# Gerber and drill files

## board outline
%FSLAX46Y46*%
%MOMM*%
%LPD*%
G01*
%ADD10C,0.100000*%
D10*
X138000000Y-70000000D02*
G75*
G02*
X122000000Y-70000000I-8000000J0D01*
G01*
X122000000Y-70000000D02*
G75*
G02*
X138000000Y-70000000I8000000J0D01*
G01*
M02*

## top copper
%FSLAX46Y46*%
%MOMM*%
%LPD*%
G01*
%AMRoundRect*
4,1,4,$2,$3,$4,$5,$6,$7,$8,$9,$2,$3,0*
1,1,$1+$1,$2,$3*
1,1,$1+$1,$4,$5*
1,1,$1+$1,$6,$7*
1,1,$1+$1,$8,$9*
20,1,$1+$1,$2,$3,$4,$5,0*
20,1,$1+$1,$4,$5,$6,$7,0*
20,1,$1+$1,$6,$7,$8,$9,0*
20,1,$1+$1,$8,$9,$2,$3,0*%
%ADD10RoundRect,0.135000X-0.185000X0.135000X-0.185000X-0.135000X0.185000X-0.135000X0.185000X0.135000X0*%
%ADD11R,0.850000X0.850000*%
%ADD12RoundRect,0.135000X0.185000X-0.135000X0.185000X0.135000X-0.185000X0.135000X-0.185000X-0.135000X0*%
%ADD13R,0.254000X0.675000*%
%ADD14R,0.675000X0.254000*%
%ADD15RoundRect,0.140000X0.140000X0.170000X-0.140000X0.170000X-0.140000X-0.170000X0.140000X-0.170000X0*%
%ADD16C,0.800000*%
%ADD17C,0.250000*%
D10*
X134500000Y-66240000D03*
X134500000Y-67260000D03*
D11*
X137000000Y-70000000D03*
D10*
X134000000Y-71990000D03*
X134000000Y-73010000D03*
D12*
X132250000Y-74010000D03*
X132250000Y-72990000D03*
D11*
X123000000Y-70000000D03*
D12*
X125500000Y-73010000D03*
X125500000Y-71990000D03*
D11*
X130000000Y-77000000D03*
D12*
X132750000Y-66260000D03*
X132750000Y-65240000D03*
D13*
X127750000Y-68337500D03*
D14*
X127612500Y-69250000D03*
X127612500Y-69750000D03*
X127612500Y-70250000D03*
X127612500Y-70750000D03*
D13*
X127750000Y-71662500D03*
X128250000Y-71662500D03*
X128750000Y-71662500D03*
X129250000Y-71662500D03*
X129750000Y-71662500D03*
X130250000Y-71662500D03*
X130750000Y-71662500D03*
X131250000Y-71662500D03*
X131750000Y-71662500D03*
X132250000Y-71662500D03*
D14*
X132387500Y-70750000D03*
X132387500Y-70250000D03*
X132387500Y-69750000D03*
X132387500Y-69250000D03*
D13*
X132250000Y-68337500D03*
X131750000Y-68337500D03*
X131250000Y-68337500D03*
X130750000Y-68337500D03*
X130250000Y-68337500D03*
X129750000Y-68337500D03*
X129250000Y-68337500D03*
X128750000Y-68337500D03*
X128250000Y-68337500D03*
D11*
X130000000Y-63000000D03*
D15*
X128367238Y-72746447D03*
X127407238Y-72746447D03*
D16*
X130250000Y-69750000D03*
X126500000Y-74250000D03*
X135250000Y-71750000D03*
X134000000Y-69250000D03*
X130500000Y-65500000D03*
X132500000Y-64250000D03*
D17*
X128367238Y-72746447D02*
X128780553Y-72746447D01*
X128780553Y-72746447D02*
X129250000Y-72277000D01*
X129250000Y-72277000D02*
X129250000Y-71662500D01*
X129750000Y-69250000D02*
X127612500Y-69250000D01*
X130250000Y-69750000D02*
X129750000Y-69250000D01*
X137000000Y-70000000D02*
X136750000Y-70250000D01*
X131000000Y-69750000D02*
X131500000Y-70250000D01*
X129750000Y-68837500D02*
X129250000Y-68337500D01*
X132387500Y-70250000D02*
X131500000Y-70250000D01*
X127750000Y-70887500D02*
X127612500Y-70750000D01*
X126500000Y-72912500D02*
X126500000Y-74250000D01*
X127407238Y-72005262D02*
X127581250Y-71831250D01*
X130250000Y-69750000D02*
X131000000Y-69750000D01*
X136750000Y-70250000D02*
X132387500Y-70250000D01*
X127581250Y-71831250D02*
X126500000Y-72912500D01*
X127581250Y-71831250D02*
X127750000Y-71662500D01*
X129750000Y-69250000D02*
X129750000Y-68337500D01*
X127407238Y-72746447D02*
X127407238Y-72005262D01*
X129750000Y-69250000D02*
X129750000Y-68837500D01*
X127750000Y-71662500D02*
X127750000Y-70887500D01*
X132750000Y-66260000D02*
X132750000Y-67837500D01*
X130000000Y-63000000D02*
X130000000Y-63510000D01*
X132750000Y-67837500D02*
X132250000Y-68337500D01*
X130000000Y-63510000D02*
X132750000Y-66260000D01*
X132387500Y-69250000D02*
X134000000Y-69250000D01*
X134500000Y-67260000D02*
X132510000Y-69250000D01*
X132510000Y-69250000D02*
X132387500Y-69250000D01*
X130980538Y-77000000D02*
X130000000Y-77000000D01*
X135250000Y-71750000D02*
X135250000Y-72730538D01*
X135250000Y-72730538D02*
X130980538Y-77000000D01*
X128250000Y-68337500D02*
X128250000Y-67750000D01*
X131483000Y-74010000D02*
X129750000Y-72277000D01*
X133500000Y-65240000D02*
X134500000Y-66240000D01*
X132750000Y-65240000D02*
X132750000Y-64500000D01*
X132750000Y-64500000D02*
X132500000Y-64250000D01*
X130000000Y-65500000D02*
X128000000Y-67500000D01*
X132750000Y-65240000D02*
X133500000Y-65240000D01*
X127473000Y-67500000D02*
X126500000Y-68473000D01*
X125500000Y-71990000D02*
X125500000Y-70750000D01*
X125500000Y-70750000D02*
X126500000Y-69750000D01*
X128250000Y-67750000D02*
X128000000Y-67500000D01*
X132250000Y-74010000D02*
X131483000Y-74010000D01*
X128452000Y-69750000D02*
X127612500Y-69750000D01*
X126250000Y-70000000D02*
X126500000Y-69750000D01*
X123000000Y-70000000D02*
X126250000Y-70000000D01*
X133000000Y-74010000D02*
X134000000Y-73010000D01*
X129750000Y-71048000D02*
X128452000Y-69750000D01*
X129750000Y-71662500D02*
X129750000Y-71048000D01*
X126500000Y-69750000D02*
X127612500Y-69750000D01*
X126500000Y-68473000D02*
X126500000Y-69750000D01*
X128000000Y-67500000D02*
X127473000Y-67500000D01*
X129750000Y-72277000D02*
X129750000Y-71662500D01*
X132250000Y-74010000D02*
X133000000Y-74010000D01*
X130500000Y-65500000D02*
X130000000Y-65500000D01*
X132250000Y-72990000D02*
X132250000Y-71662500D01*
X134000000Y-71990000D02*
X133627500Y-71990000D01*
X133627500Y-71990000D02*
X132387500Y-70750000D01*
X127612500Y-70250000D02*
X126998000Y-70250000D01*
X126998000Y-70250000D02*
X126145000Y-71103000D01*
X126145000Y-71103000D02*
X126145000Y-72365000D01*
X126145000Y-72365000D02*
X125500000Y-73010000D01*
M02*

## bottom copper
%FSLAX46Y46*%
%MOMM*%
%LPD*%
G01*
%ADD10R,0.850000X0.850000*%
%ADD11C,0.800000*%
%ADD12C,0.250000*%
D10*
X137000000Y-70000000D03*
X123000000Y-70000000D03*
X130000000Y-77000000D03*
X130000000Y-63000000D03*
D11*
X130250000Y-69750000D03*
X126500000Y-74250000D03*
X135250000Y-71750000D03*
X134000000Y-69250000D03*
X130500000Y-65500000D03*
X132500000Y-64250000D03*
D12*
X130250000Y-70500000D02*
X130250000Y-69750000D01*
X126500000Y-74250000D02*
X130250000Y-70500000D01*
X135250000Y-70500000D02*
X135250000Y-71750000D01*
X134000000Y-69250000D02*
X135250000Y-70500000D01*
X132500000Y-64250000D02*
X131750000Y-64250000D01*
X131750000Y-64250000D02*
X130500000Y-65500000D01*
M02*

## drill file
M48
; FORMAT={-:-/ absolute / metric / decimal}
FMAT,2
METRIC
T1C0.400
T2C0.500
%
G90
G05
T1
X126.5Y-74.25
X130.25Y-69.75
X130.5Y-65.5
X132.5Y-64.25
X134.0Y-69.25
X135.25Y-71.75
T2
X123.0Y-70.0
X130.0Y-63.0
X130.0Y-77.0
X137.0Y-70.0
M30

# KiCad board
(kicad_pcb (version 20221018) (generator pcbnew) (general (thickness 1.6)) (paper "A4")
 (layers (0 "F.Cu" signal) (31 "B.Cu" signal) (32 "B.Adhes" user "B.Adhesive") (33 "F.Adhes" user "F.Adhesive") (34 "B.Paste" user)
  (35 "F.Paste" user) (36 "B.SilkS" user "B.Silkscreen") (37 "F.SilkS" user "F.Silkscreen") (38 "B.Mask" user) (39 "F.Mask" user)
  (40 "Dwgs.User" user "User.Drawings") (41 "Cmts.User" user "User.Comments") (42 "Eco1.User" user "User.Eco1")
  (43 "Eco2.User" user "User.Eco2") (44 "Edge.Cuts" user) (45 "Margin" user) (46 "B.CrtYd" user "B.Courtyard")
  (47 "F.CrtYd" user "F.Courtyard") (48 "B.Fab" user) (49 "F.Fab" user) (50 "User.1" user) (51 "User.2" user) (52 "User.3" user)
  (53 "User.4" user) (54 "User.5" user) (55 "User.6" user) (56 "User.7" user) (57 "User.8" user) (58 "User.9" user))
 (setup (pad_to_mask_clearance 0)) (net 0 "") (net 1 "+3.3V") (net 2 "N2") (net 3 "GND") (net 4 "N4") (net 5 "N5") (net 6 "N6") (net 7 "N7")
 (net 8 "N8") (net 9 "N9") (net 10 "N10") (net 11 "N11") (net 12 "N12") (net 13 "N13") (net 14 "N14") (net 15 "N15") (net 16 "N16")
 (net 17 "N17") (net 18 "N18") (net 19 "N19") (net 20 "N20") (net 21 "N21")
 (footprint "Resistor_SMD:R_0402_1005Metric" (layer "F.Cu") (at 134.5 66.75 -90)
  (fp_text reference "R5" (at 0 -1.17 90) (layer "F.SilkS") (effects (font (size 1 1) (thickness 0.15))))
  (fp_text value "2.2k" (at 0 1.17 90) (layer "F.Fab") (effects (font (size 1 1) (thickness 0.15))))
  (pad "1" smd roundrect (at -0.51 0 270) (size 0.54 0.64) (layers "F.Cu" "F.Paste" "F.Mask") (roundrect_rratio 0.25) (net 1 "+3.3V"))
  (pad "2" smd roundrect (at 0.51 0 270) (size 0.54 0.64) (layers "F.Cu" "F.Paste" "F.Mask") (roundrect_rratio 0.25) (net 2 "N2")))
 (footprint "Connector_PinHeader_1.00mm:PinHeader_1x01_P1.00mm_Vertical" (layer "F.Cu") (at 137 70 -90)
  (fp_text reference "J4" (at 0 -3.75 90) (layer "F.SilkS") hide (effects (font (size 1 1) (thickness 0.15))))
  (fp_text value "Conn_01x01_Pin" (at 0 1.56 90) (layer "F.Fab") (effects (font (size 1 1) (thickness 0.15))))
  (pad "1" thru_hole rect (at 0 0 270) (size 0.85 0.85) (drill 0.5) (layers "*.Cu" "*.Mask") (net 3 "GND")))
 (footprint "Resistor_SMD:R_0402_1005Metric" (layer "F.Cu") (at 134 72.5 -90)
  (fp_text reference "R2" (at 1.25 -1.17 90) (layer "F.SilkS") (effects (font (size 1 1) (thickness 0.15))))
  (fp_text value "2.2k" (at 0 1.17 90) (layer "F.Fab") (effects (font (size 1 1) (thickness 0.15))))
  (pad "1" smd roundrect (at -0.51 0 270) (size 0.54 0.64) (layers "F.Cu" "F.Paste" "F.Mask") (roundrect_rratio 0.25) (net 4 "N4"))
  (pad "2" smd roundrect (at 0.51 0 270) (size 0.54 0.64) (layers "F.Cu" "F.Paste" "F.Mask") (roundrect_rratio 0.25) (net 1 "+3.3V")))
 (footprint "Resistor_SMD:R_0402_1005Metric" (layer "F.Cu") (at 132.25 73.5 90)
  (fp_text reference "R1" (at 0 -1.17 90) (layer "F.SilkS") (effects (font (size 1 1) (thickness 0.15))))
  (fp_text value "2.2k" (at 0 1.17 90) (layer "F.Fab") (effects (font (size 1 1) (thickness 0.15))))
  (pad "1" smd roundrect (at -0.51 0 90) (size 0.54 0.64) (layers "F.Cu" "F.Paste" "F.Mask") (roundrect_rratio 0.25) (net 1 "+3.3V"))
  (pad "2" smd roundrect (at 0.51 0 90) (size 0.54 0.64) (layers "F.Cu" "F.Paste" "F.Mask") (roundrect_rratio 0.25) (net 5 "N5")))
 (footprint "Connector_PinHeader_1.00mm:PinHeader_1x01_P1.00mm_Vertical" (layer "F.Cu") (at 123 70 90)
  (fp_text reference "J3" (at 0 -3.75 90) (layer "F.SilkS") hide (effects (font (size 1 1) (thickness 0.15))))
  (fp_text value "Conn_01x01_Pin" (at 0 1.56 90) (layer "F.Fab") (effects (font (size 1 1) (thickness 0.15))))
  (pad "1" thru_hole rect (at 0 0 90) (size 0.85 0.85) (drill 0.5) (layers "*.Cu" "*.Mask") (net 1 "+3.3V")))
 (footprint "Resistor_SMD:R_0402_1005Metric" (layer "F.Cu") (at 125.5 72.5 90)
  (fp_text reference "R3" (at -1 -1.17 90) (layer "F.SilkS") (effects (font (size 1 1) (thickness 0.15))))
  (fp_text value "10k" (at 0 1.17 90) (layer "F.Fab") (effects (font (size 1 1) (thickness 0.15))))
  (pad "1" smd roundrect (at -0.51 0 90) (size 0.54 0.64) (layers "F.Cu" "F.Paste" "F.Mask") (roundrect_rratio 0.25) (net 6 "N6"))
  (pad "2" smd roundrect (at 0.51 0 90) (size 0.54 0.64) (layers "F.Cu" "F.Paste" "F.Mask") (roundrect_rratio 0.25) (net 1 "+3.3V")))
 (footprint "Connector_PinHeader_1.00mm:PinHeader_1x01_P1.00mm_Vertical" (layer "F.Cu") (at 130 77 180)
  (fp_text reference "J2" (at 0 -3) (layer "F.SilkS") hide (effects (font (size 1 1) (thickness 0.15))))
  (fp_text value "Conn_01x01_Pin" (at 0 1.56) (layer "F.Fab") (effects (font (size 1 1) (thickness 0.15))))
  (pad "1" thru_hole rect (at 0 0 180) (size 0.85 0.85) (drill 0.5) (layers "*.Cu" "*.Mask") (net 2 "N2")))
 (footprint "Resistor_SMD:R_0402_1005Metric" (layer "F.Cu") (at 132.75 65.75 90)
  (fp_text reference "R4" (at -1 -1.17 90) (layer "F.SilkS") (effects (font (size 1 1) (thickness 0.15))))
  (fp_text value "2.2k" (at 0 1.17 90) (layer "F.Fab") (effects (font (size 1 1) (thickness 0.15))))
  (pad "1" smd roundrect (at -0.51 0 90) (size 0.54 0.64) (layers "F.Cu" "F.Paste" "F.Mask") (roundrect_rratio 0.25) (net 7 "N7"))
  (pad "2" smd roundrect (at 0.51 0 90) (size 0.54 0.64) (layers "F.Cu" "F.Paste" "F.Mask") (roundrect_rratio 0.25) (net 1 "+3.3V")))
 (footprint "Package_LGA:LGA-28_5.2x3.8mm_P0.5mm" (layer "F.Cu") (at 130 70)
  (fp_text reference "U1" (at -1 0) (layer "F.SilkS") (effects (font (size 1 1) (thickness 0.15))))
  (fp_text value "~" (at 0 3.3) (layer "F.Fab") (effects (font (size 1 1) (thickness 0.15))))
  (pad "1" smd rect (at -2.25 -1.6625) (size 0.254 0.675) (layers "F.Cu" "F.Paste" "F.Mask") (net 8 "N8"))
  (pad "2" smd rect (at -2.3875 -0.75 90) (size 0.254 0.675) (layers "F.Cu" "F.Paste" "F.Mask") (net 3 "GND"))
  (pad "3" smd rect (at -2.3875 -0.25 90) (size 0.254 0.675) (layers "F.Cu" "F.Paste" "F.Mask") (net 1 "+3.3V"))
  (pad "4" smd rect (at -2.3875 0.25 90) (size 0.254 0.675) (layers "F.Cu" "F.Paste" "F.Mask") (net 6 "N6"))
  (pad "5" smd rect (at -2.3875 0.75 90) (size 0.254 0.675) (layers "F.Cu" "F.Paste" "F.Mask") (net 3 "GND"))
  (pad "6" smd rect (at -2.25 1.6625) (size 0.254 0.675) (layers "F.Cu" "F.Paste" "F.Mask") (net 3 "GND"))
  (pad "7" smd rect (at -1.75 1.6625) (size 0.254 0.675) (layers "F.Cu" "F.Paste" "F.Mask") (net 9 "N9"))
  (pad "8" smd rect (at -1.25 1.6625) (size 0.254 0.675) (layers "F.Cu" "F.Paste" "F.Mask") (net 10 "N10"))
  (pad "9" smd rect (at -0.75 1.6625) (size 0.254 0.675) (layers "F.Cu" "F.Paste" "F.Mask") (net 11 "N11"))
  (pad "10" smd rect (at -0.25 1.6625) (size 0.254 0.675) (layers "F.Cu" "F.Paste" "F.Mask") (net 1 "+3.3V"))
  (pad "11" smd rect (at 0.25 1.6625) (size 0.254 0.675) (layers "F.Cu" "F.Paste" "F.Mask") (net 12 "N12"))
  (pad "12" smd rect (at 0.75 1.6625) (size 0.254 0.675) (layers "F.Cu" "F.Paste" "F.Mask") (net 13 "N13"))
  (pad "13" smd rect (at 1.25 1.6625) (size 0.254 0.675) (layers "F.Cu" "F.Paste" "F.Mask") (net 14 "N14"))
  (pad "14" smd rect (at 1.75 1.6625) (size 0.254 0.675) (layers "F.Cu" "F.Paste" "F.Mask") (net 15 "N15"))
  (pad "15" smd rect (at 2.25 1.6625) (size 0.254 0.675) (layers "F.Cu" "F.Paste" "F.Mask") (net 5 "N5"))
  (pad "16" smd rect (at 2.3875 0.75 90) (size 0.254 0.675) (layers "F.Cu" "F.Paste" "F.Mask") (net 4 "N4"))
  (pad "17" smd rect (at 2.3875 0.25 90) (size 0.254 0.675) (layers "F.Cu" "F.Paste" "F.Mask") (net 3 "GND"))
  (pad "18" smd rect (at 2.3875 -0.25 90) (size 0.254 0.675) (layers "F.Cu" "F.Paste" "F.Mask") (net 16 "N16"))
  (pad "19" smd rect (at 2.3875 -0.75 90) (size 0.254 0.675) (layers "F.Cu" "F.Paste" "F.Mask") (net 2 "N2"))
  (pad "20" smd rect (at 2.25 -1.6625) (size 0.254 0.675) (layers "F.Cu" "F.Paste" "F.Mask") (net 7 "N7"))
  (pad "21" smd rect (at 1.75 -1.6625) (size 0.254 0.675) (layers "F.Cu" "F.Paste" "F.Mask") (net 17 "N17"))
  (pad "22" smd rect (at 1.25 -1.6625) (size 0.254 0.675) (layers "F.Cu" "F.Paste" "F.Mask") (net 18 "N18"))
  (pad "23" smd rect (at 0.75 -1.6625) (size 0.254 0.675) (layers "F.Cu" "F.Paste" "F.Mask") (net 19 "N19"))
  (pad "24" smd rect (at 0.25 -1.6625) (size 0.254 0.675) (layers "F.Cu" "F.Paste" "F.Mask") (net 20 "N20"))
  (pad "25" smd rect (at -0.25 -1.6625) (size 0.254 0.675) (layers "F.Cu" "F.Paste" "F.Mask") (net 3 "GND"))
  (pad "26" smd rect (at -0.75 -1.6625) (size 0.254 0.675) (layers "F.Cu" "F.Paste" "F.Mask") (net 3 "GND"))
  (pad "27" smd rect (at -1.25 -1.6625) (size 0.254 0.675) (layers "F.Cu" "F.Paste" "F.Mask") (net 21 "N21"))
  (pad "28" smd rect (at -1.75 -1.6625) (size 0.254 0.675) (layers "F.Cu" "F.Paste" "F.Mask") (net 1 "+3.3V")))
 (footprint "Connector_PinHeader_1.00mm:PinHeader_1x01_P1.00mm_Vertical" (layer "F.Cu") (at 130 63)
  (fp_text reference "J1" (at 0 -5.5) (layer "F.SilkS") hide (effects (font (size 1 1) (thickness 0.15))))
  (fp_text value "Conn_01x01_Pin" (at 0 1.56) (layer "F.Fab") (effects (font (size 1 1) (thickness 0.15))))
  (pad "1" thru_hole rect (at 0 0) (size 0.85 0.85) (drill 0.5) (layers "*.Cu" "*.Mask") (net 7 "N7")))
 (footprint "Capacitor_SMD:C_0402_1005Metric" (layer "F.Cu") (at 127.887238 72.746447 180)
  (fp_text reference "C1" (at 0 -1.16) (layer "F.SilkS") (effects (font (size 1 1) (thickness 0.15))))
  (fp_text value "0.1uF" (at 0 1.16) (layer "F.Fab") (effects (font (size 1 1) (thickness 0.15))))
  (pad "1" smd roundrect (at -0.48 0 180) (size 0.56 0.62) (layers "F.Cu" "F.Paste" "F.Mask") (roundrect_rratio 0.25) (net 11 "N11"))
  (pad "2" smd roundrect (at 0.48 0 180) (size 0.56 0.62) (layers "F.Cu" "F.Paste" "F.Mask") (roundrect_rratio 0.25) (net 3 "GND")))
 (gr_circle (center 130 70) (end 138 70) (stroke (width 0.1) (type default)) (fill none) (layer "Edge.Cuts"))
 (segment (start 128.367238 72.746447) (end 128.780553 72.746447) (width 0.25) (layer "F.Cu") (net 11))
 (segment (start 128.780553 72.746447) (end 129.25 72.277) (width 0.25) (layer "F.Cu") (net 11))
 (segment (start 129.25 72.277) (end 129.25 71.6625) (width 0.25) (layer "F.Cu") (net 11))
 (segment (start 129.75 69.25) (end 127.6125 69.25) (width 0.25) (layer "F.Cu") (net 3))
 (segment (start 130.25 69.75) (end 129.75 69.25) (width 0.25) (layer "F.Cu") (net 3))
 (segment (start 137 70) (end 136.75 70.25) (width 0.25) (layer "F.Cu") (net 3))
 (segment (start 131 69.75) (end 131.5 70.25) (width 0.25) (layer "F.Cu") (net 3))
 (segment (start 129.75 68.8375) (end 129.25 68.3375) (width 0.25) (layer "F.Cu") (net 3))
 (segment (start 132.3875 70.25) (end 131.5 70.25) (width 0.25) (layer "F.Cu") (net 3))
 (segment (start 127.75 70.8875) (end 127.6125 70.75) (width 0.25) (layer "F.Cu") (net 3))
 (segment (start 126.5 72.9125) (end 126.5 74.25) (width 0.25) (layer "F.Cu") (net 3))
 (segment (start 127.407238 72.005262) (end 127.58125 71.83125) (width 0.25) (layer "F.Cu") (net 3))
 (segment (start 130.25 69.75) (end 131 69.75) (width 0.25) (layer "F.Cu") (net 3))
 (segment (start 136.75 70.25) (end 132.3875 70.25) (width 0.25) (layer "F.Cu") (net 3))
 (segment (start 127.58125 71.83125) (end 126.5 72.9125) (width 0.25) (layer "F.Cu") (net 3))
 (segment (start 127.58125 71.83125) (end 127.75 71.6625) (width 0.25) (layer "F.Cu") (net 3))
 (segment (start 129.75 69.25) (end 129.75 68.3375) (width 0.25) (layer "F.Cu") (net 3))
 (segment (start 127.407238 72.746447) (end 127.407238 72.005262) (width 0.25) (layer "F.Cu") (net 3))
 (segment (start 129.75 69.25) (end 129.75 68.8375) (width 0.25) (layer "F.Cu") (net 3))
 (segment (start 127.75 71.6625) (end 127.75 70.8875) (width 0.25) (layer "F.Cu") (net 3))
 (via (at 130.25 69.75) (size 0.8) (drill 0.4) (layers "F.Cu" "B.Cu") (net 3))
 (via (at 126.5 74.25) (size 0.8) (drill 0.4) (layers "F.Cu" "B.Cu") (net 3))
 (segment (start 130.25 70.5) (end 130.25 69.75) (width 0.25) (layer "B.Cu") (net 3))
 (segment (start 126.5 74.25) (end 130.25 70.5) (width 0.25) (layer "B.Cu") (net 3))
 (segment (start 132.75 66.26) (end 132.75 67.8375) (width 0.25) (layer "F.Cu") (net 7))
 (segment (start 130 63) (end 130 63.51) (width 0.25) (layer "F.Cu") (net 7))
 (segment (start 132.75 67.8375) (end 132.25 68.3375) (width 0.25) (layer "F.Cu") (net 7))
 (segment (start 130 63.51) (end 132.75 66.26) (width 0.25) (layer "F.Cu") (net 7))
 (segment (start 132.3875 69.25) (end 134 69.25) (width 0.25) (layer "F.Cu") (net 2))
 (segment (start 134.5 67.26) (end 132.51 69.25) (width 0.25) (layer "F.Cu") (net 2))
 (segment (start 132.51 69.25) (end 132.3875 69.25) (width 0.25) (layer "F.Cu") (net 2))
 (segment (start 130.980538 77) (end 130 77) (width 0.25) (layer "F.Cu") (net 2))
 (segment (start 135.25 71.75) (end 135.25 72.730538) (width 0.25) (layer "F.Cu") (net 2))
 (segment (start 135.25 72.730538) (end 130.980538 77) (width 0.25) (layer "F.Cu") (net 2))
 (via (at 135.25 71.75) (size 0.8) (drill 0.4) (layers "F.Cu" "B.Cu") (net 2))
 (via (at 134 69.25) (size 0.8) (drill 0.4) (layers "F.Cu" "B.Cu") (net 2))
 (segment (start 135.25 70.5) (end 135.25 71.75) (width 0.25) (layer "B.Cu") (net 2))
 (segment (start 134 69.25) (end 135.25 70.5) (width 0.25) (layer "B.Cu") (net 2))
 (segment (start 128.25 68.3375) (end 128.25 67.75) (width 0.25) (layer "F.Cu") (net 1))
 (segment (start 131.483 74.01) (end 129.75 72.277) (width 0.25) (layer "F.Cu") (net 1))
 (segment (start 133.5 65.24) (end 134.5 66.24) (width 0.25) (layer "F.Cu") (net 1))
 (segment (start 132.75 65.24) (end 132.75 64.5) (width 0.25) (layer "F.Cu") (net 1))
 (segment (start 132.75 64.5) (end 132.5 64.25) (width 0.25) (layer "F.Cu") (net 1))
 (segment (start 130 65.5) (end 128 67.5) (width 0.25) (layer "F.Cu") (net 1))
 (segment (start 132.75 65.24) (end 133.5 65.24) (width 0.25) (layer "F.Cu") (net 1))
 (segment (start 127.473 67.5) (end 126.5 68.473) (width 0.25) (layer "F.Cu") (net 1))
 (segment (start 125.5 71.99) (end 125.5 70.75) (width 0.25) (layer "F.Cu") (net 1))
 (segment (start 125.5 70.75) (end 126.5 69.75) (width 0.25) (layer "F.Cu") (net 1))
 (segment (start 128.25 67.75) (end 128 67.5) (width 0.25) (layer "F.Cu") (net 1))
 (segment (start 132.25 74.01) (end 131.483 74.01) (width 0.25) (layer "F.Cu") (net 1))
 (segment (start 128.452 69.75) (end 127.6125 69.75) (width 0.25) (layer "F.Cu") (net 1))
 (segment (start 126.25 70) (end 126.5 69.75) (width 0.25) (layer "F.Cu") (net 1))
 (segment (start 123 70) (end 126.25 70) (width 0.25) (layer "F.Cu") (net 1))
 (segment (start 133 74.01) (end 134 73.01) (width 0.25) (layer "F.Cu") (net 1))
 (segment (start 129.75 71.048) (end 128.452 69.75) (width 0.25) (layer "F.Cu") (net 1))
 (segment (start 129.75 71.6625) (end 129.75 71.048) (width 0.25) (layer "F.Cu") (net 1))
 (segment (start 126.5 69.75) (end 127.6125 69.75) (width 0.25) (layer "F.Cu") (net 1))
 (segment (start 126.5 68.473) (end 126.5 69.75) (width 0.25) (layer "F.Cu") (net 1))
 (segment (start 128 67.5) (end 127.473 67.5) (width 0.25) (layer "F.Cu") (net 1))
 (segment (start 129.75 72.277) (end 129.75 71.6625) (width 0.25) (layer "F.Cu") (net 1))
 (segment (start 132.25 74.01) (end 133 74.01) (width 0.25) (layer "F.Cu") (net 1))
 (segment (start 130.5 65.5) (end 130 65.5) (width 0.25) (layer "F.Cu") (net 1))
 (via (at 130.5 65.5) (size 0.8) (drill 0.4) (layers "F.Cu" "B.Cu") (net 1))
 (via (at 132.5 64.25) (size 0.8) (drill 0.4) (layers "F.Cu" "B.Cu") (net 1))
 (segment (start 132.5 64.25) (end 131.75 64.25) (width 0.25) (layer "B.Cu") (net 1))
 (segment (start 131.75 64.25) (end 130.5 65.5) (width 0.25) (layer "B.Cu") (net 1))
 (segment (start 132.25 72.99) (end 132.25 71.6625) (width 0.25) (layer "F.Cu") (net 5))
 (segment (start 134 71.99) (end 133.6275 71.99) (width 0.25) (layer "F.Cu") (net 4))
 (segment (start 133.6275 71.99) (end 132.3875 70.75) (width 0.25) (layer "F.Cu") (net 4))
 (segment (start 127.6125 70.25) (end 126.998 70.25) (width 0.25) (layer "F.Cu") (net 6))
 (segment (start 126.998 70.25) (end 126.145 71.103) (width 0.25) (layer "F.Cu") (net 6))
 (segment (start 126.145 71.103) (end 126.145 72.365) (width 0.25) (layer "F.Cu") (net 6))
 (segment (start 126.145 72.365) (end 125.5 73.01) (width 0.25) (layer "F.Cu") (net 6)))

